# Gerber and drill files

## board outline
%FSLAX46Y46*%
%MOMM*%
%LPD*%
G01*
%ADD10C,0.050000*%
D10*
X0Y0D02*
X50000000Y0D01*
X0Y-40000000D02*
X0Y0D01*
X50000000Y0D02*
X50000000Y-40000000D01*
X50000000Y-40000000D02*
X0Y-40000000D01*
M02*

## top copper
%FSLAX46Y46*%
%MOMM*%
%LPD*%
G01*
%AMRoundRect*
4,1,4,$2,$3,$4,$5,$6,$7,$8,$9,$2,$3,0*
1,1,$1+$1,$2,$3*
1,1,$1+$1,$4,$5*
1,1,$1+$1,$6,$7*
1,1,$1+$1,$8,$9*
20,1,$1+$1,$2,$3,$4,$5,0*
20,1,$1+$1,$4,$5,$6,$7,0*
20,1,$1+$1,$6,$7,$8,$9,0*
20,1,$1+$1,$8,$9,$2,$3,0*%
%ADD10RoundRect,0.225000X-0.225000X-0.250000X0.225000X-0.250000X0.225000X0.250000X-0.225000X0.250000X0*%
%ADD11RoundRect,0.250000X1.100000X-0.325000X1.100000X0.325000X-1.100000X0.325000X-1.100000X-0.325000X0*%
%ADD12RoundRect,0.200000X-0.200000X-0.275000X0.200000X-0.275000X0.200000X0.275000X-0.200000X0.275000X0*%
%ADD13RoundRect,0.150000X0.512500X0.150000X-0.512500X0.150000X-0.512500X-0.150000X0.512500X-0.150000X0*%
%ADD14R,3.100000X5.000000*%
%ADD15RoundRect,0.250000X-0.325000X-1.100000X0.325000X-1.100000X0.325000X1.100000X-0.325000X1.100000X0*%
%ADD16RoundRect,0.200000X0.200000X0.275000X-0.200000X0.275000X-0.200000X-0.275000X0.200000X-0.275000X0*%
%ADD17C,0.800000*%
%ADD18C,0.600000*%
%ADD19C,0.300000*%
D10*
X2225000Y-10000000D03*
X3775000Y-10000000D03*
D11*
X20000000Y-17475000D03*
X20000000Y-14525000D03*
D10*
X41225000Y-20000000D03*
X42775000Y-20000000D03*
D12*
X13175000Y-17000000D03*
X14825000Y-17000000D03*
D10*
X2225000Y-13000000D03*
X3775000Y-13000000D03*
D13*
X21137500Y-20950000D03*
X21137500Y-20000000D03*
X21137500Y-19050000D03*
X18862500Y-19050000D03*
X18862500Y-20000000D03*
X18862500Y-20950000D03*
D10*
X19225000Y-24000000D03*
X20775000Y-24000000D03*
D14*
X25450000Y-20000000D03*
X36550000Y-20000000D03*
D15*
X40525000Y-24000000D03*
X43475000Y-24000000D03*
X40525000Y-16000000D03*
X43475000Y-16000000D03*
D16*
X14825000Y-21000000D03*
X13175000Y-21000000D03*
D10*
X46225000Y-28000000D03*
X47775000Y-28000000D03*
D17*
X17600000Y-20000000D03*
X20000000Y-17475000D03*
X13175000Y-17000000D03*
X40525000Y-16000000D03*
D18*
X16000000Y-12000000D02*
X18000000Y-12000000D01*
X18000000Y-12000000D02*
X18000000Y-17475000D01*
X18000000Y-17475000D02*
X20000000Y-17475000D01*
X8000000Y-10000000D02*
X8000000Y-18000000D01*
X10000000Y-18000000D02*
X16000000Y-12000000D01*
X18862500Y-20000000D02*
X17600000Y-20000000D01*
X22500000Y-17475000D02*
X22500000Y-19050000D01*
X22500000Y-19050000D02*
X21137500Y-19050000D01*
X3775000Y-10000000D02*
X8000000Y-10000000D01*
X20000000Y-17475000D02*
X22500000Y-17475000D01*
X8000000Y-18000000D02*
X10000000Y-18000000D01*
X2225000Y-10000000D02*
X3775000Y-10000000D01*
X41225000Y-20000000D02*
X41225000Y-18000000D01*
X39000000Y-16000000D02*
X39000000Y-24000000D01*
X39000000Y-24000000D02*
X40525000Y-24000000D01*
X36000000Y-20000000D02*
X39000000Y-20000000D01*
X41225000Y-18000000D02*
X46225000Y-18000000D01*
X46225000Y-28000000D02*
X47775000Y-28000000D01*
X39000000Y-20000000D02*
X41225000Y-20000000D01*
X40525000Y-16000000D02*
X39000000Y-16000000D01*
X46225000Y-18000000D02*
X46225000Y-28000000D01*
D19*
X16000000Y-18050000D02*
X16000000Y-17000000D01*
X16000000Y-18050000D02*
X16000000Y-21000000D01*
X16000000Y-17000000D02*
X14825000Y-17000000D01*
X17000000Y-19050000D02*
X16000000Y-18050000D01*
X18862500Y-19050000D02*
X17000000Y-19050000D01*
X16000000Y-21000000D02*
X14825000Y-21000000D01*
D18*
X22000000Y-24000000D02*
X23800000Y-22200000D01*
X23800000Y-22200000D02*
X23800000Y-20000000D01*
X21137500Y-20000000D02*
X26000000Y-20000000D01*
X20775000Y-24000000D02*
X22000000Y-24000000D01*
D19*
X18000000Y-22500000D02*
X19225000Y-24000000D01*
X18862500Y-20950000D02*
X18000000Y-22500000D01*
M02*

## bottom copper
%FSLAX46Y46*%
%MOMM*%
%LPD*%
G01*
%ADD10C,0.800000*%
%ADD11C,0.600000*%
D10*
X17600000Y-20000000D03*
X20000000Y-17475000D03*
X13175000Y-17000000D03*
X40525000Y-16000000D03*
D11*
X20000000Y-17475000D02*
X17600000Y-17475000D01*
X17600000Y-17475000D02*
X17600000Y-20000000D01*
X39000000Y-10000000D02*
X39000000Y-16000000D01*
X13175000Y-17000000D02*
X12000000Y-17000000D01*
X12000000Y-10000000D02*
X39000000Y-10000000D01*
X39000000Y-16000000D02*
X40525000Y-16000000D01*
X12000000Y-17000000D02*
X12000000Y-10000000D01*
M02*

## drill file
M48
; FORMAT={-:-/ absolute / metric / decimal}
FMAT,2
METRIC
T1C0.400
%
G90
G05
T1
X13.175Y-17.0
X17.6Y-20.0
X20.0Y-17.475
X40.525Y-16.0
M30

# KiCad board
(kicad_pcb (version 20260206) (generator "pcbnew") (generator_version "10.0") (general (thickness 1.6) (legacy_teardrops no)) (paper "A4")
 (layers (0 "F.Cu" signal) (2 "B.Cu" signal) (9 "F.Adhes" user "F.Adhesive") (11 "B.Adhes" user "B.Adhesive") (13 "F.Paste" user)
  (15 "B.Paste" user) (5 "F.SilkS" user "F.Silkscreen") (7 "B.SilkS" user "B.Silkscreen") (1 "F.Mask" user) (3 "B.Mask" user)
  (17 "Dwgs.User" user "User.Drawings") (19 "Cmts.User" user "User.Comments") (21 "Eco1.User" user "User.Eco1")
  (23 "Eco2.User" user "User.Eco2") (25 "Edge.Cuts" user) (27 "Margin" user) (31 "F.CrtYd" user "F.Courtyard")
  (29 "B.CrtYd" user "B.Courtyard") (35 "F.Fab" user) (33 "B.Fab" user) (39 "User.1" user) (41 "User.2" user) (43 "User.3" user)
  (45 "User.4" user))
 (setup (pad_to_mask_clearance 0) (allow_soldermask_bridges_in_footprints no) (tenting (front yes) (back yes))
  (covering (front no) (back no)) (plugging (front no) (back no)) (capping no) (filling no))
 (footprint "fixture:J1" (layer "F.Cu") (at 3 10)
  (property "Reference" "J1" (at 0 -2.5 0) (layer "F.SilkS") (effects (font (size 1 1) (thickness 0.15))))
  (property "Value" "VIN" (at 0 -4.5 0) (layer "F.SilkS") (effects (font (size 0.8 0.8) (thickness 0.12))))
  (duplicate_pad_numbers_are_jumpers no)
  (pad "1" smd roundrect (at -0.775 0) (size 0.9 0.95) (layers "F.Cu" "F.Mask" "F.Paste") (roundrect_rratio 0.25) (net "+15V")
   (thermal_bridge_angle 45))
  (pad "2" smd roundrect (at 0.775 0) (size 0.9 0.95) (layers "F.Cu" "F.Mask" "F.Paste") (roundrect_rratio 0.25) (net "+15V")
   (thermal_bridge_angle 45)))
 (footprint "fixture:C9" (layer "F.Cu") (at 20 16 90)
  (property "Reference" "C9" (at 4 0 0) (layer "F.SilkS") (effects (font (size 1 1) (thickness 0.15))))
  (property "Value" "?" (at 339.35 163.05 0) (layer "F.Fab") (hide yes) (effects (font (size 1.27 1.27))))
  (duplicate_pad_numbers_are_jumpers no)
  (pad "1" smd roundrect (at -1.475 0 90) (size 1.15 2.7) (layers "F.Cu" "F.Mask" "F.Paste") (roundrect_rratio 0.217391) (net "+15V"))
  (pad "2" smd roundrect (at 1.475 0 90) (size 1.15 2.7) (layers "F.Cu" "F.Mask" "F.Paste") (roundrect_rratio 0.217391) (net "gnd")))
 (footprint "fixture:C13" (layer "F.Cu") (at 42 20)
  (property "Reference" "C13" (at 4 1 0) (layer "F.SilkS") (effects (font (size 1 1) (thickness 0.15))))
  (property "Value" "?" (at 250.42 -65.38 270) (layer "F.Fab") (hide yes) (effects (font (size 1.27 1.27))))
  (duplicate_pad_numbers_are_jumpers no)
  (pad "1" smd roundrect (at -0.775 0) (size 0.9 0.95) (layers "F.Cu" "F.Mask" "F.Paste") (roundrect_rratio 0.25) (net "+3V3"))
  (pad "2" smd roundrect (at 0.775 0) (size 0.9 0.95) (layers "F.Cu" "F.Mask" "F.Paste") (roundrect_rratio 0.25) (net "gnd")))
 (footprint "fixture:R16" (layer "F.Cu") (at 14 17)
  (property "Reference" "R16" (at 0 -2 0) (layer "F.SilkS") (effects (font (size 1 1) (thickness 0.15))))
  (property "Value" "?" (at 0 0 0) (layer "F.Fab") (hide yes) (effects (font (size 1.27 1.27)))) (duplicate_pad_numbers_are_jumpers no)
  (pad "1" smd roundrect (at -0.825 0) (size 0.8 0.95) (layers "F.Cu" "F.Mask" "F.Paste") (roundrect_rratio 0.25) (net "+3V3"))
  (pad "2" smd roundrect (at 0.825 0) (size 0.8 0.95) (layers "F.Cu" "F.Mask" "F.Paste") (roundrect_rratio 0.25) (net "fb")))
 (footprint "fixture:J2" (layer "F.Cu") (at 3 13)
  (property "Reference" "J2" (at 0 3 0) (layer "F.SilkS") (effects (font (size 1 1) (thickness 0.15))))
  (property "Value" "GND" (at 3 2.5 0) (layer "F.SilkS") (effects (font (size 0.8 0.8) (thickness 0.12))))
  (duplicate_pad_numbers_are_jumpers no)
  (pad "1" smd roundrect (at -0.775 0) (size 0.9 0.95) (layers "F.Cu" "F.Mask" "F.Paste") (roundrect_rratio 0.25) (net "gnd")
   (thermal_bridge_angle 45))
  (pad "2" smd roundrect (at 0.775 0) (size 0.9 0.95) (layers "F.Cu" "F.Mask" "F.Paste") (roundrect_rratio 0.25) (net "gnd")
   (thermal_bridge_angle 45)))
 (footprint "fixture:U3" (layer "F.Cu") (at 20 20 180)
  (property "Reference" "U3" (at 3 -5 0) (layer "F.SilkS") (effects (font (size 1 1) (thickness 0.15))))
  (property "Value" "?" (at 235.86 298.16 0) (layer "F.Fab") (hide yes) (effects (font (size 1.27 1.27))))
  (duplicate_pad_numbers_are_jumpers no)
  (pad "1" smd roundrect (at -1.1375 -0.95 180) (size 1.325 0.6) (layers "F.Cu" "F.Mask" "F.Paste") (roundrect_rratio 0.25) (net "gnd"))
  (pad "2" smd roundrect (at -1.1375 0 180) (size 1.325 0.6) (layers "F.Cu" "F.Mask" "F.Paste") (roundrect_rratio 0.25) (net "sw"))
  (pad "3" smd roundrect (at -1.1375 0.95 180) (size 1.325 0.6) (layers "F.Cu" "F.Mask" "F.Paste") (roundrect_rratio 0.25) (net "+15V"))
  (pad "4" smd roundrect (at 1.1375 0.95 180) (size 1.325 0.6) (layers "F.Cu" "F.Mask" "F.Paste") (roundrect_rratio 0.25) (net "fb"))
  (pad "5" smd roundrect (at 1.1375 0 180) (size 1.325 0.6) (layers "F.Cu" "F.Mask" "F.Paste") (roundrect_rratio 0.25) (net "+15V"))
  (pad "6" smd roundrect (at 1.1375 -0.95 180) (size 1.325 0.6) (layers "F.Cu" "F.Mask" "F.Paste") (roundrect_rratio 0.25) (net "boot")))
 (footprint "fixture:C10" (layer "F.Cu") (at 20 24)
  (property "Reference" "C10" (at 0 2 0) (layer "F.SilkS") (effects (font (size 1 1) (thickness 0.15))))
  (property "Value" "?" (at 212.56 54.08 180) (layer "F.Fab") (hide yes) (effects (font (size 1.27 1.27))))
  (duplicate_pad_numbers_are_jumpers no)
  (pad "1" smd roundrect (at -0.775 0) (size 0.9 0.95) (layers "F.Cu" "F.Mask" "F.Paste") (roundrect_rratio 0.25) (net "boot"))
  (pad "2" smd roundrect (at 0.775 0) (size 0.9 0.95) (layers "F.Cu" "F.Mask" "F.Paste") (roundrect_rratio 0.25) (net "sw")))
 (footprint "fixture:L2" (layer "F.Cu") (at 31 20)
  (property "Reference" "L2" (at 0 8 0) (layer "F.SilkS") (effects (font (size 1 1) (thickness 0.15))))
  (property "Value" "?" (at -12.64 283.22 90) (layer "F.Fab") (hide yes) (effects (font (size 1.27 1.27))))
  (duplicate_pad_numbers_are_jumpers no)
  (pad "1" smd rect (at -5.55 0) (size 3.1 5) (layers "F.Cu" "F.Mask" "F.Paste") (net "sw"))
  (pad "2" smd rect (at 5.55 0) (size 3.1 5) (layers "F.Cu" "F.Mask" "F.Paste") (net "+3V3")))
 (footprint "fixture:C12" (layer "F.Cu") (at 42 24)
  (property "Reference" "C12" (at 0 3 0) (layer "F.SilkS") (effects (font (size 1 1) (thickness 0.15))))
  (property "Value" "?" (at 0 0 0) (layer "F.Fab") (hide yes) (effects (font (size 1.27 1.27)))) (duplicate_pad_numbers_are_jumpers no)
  (pad "1" smd roundrect (at -1.475 0) (size 1.15 2.7) (layers "F.Cu" "F.Mask" "F.Paste") (roundrect_rratio 0.217391) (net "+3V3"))
  (pad "2" smd roundrect (at 1.475 0) (size 1.15 2.7) (layers "F.Cu" "F.Mask" "F.Paste") (roundrect_rratio 0.217391) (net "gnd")))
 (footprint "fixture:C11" (layer "F.Cu") (at 42 16)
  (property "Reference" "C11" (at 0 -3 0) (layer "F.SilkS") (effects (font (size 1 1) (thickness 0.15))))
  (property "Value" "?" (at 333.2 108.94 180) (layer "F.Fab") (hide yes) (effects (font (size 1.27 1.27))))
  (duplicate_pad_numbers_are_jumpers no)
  (pad "1" smd roundrect (at -1.475 0) (size 1.15 2.7) (layers "F.Cu" "F.Mask" "F.Paste") (roundrect_rratio 0.217391) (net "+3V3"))
  (pad "2" smd roundrect (at 1.475 0) (size 1.15 2.7) (layers "F.Cu" "F.Mask" "F.Paste") (roundrect_rratio 0.217391) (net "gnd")))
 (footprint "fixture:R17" (layer "F.Cu") (at 14 21 180)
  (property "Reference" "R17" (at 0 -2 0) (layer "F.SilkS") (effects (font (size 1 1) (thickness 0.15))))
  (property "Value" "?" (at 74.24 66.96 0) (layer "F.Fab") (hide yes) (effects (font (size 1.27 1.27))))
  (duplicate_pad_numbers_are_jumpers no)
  (pad "1" smd roundrect (at -0.825 0 180) (size 0.8 0.95) (layers "F.Cu" "F.Mask" "F.Paste") (roundrect_rratio 0.25) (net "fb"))
  (pad "2" smd roundrect (at 0.825 0 180) (size 0.8 0.95) (layers "F.Cu" "F.Mask" "F.Paste") (roundrect_rratio 0.25) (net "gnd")))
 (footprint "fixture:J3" (layer "F.Cu") (at 47 28)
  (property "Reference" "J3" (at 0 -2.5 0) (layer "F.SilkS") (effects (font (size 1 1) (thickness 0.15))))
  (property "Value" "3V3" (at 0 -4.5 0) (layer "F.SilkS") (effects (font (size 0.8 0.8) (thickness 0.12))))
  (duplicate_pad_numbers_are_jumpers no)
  (pad "1" smd roundrect (at -0.775 0) (size 0.9 0.95) (layers "F.Cu" "F.Mask" "F.Paste") (roundrect_rratio 0.25) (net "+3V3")
   (thermal_bridge_angle 45))
  (pad "2" smd roundrect (at 0.775 0) (size 0.9 0.95) (layers "F.Cu" "F.Mask" "F.Paste") (roundrect_rratio 0.25) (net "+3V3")
   (thermal_bridge_angle 45)))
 (gr_line (start 0 0) (end 50 0) (stroke (width 0.05) (type default)) (layer "Edge.Cuts"))
 (gr_line (start 0 40) (end 0 0) (stroke (width 0.05) (type default)) (layer "Edge.Cuts"))
 (gr_line (start 50 0) (end 50 40) (stroke (width 0.05) (type default)) (layer "Edge.Cuts"))
 (gr_line (start 50 40) (end 0 40) (stroke (width 0.05) (type default)) (layer "Edge.Cuts"))
 (segment (start 16 12) (end 18 12) (width 0.6) (layer "F.Cu") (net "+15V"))
 (segment (start 18 12) (end 18 17.475) (width 0.6) (layer "F.Cu") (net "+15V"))
 (segment (start 18 17.475) (end 20 17.475) (width 0.6) (layer "F.Cu") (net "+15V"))
 (segment (start 8 10) (end 8 18) (width 0.6) (layer "F.Cu") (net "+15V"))
 (segment (start 10 18) (end 16 12) (width 0.6) (layer "F.Cu") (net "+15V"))
 (segment (start 18.8625 20) (end 17.6 20) (width 0.6) (layer "F.Cu") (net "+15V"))
 (segment (start 22.5 17.475) (end 22.5 19.05) (width 0.6) (layer "F.Cu") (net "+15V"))
 (segment (start 22.5 19.05) (end 21.1375 19.05) (width 0.6) (layer "F.Cu") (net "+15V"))
 (segment (start 3.775 10) (end 8 10) (width 0.6) (layer "F.Cu") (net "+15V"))
 (segment (start 20 17.475) (end 22.5 17.475) (width 0.6) (layer "F.Cu") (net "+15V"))
 (segment (start 8 18) (end 10 18) (width 0.6) (layer "F.Cu") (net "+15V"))
 (segment (start 2.225 10) (end 3.775 10) (width 0.6) (layer "F.Cu") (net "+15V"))
 (via (at 17.6 20) (size 0.8) (drill 0.4) (layers "F.Cu" "B.Cu") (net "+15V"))
 (via (at 20 17.475) (size 0.8) (drill 0.4) (layers "F.Cu" "B.Cu") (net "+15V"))
 (segment (start 20 17.475) (end 17.6 17.475) (width 0.6) (layer "B.Cu") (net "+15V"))
 (segment (start 17.6 17.475) (end 17.6 20) (width 0.6) (layer "B.Cu") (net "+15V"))
 (segment (start 41.225 20) (end 41.225 18) (width 0.6) (layer "F.Cu") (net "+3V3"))
 (segment (start 39 16) (end 39 24) (width 0.6) (layer "F.Cu") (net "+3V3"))
 (segment (start 39 24) (end 40.525 24) (width 0.6) (layer "F.Cu") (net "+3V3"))
 (segment (start 36 20) (end 39 20) (width 0.6) (layer "F.Cu") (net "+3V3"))
 (segment (start 41.225 18) (end 46.225 18) (width 0.6) (layer "F.Cu") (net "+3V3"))
 (segment (start 46.225 28) (end 47.775 28) (width 0.6) (layer "F.Cu") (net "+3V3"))
 (segment (start 39 20) (end 41.225 20) (width 0.6) (layer "F.Cu") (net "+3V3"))
 (segment (start 40.525 16) (end 39 16) (width 0.6) (layer "F.Cu") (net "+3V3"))
 (segment (start 46.225 18) (end 46.225 28) (width 0.6) (layer "F.Cu") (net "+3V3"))
 (via (at 13.175 17) (size 0.8) (drill 0.4) (layers "F.Cu" "B.Cu") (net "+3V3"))
 (via (at 40.525 16) (size 0.8) (drill 0.4) (layers "F.Cu" "B.Cu") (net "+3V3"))
 (segment (start 39 10) (end 39 16) (width 0.6) (layer "B.Cu") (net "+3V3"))
 (segment (start 13.175 17) (end 12 17) (width 0.6) (layer "B.Cu") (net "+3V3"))
 (segment (start 12 10) (end 39 10) (width 0.6) (layer "B.Cu") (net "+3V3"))
 (segment (start 39 16) (end 40.525 16) (width 0.6) (layer "B.Cu") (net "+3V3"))
 (segment (start 12 17) (end 12 10) (width 0.6) (layer "B.Cu") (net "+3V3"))
 (segment (start 16 18.05) (end 16 17) (width 0.3) (layer "F.Cu") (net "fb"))
 (segment (start 16 18.05) (end 16 21) (width 0.3) (layer "F.Cu") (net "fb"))
 (segment (start 16 17) (end 14.825 17) (width 0.3) (layer "F.Cu") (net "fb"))
 (segment (start 17 19.05) (end 16 18.05) (width 0.3) (layer "F.Cu") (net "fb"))
 (segment (start 18.8625 19.05) (end 17 19.05) (width 0.3) (layer "F.Cu") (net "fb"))
 (segment (start 16 21) (end 14.825 21) (width 0.3) (layer "F.Cu") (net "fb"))
 (segment (start 22 24) (end 23.8 22.2) (width 0.6) (layer "F.Cu") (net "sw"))
 (segment (start 23.8 22.2) (end 23.8 20) (width 0.6) (layer "F.Cu") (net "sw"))
 (segment (start 21.1375 20) (end 26 20) (width 0.6) (layer "F.Cu") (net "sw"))
 (segment (start 20.775 24) (end 22 24) (width 0.6) (layer "F.Cu") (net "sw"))
 (segment (start 18 22.5) (end 19.225 24) (width 0.3) (layer "F.Cu") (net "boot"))
 (segment (start 18.8625 20.95) (end 18 22.5) (width 0.3) (layer "F.Cu") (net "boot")))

